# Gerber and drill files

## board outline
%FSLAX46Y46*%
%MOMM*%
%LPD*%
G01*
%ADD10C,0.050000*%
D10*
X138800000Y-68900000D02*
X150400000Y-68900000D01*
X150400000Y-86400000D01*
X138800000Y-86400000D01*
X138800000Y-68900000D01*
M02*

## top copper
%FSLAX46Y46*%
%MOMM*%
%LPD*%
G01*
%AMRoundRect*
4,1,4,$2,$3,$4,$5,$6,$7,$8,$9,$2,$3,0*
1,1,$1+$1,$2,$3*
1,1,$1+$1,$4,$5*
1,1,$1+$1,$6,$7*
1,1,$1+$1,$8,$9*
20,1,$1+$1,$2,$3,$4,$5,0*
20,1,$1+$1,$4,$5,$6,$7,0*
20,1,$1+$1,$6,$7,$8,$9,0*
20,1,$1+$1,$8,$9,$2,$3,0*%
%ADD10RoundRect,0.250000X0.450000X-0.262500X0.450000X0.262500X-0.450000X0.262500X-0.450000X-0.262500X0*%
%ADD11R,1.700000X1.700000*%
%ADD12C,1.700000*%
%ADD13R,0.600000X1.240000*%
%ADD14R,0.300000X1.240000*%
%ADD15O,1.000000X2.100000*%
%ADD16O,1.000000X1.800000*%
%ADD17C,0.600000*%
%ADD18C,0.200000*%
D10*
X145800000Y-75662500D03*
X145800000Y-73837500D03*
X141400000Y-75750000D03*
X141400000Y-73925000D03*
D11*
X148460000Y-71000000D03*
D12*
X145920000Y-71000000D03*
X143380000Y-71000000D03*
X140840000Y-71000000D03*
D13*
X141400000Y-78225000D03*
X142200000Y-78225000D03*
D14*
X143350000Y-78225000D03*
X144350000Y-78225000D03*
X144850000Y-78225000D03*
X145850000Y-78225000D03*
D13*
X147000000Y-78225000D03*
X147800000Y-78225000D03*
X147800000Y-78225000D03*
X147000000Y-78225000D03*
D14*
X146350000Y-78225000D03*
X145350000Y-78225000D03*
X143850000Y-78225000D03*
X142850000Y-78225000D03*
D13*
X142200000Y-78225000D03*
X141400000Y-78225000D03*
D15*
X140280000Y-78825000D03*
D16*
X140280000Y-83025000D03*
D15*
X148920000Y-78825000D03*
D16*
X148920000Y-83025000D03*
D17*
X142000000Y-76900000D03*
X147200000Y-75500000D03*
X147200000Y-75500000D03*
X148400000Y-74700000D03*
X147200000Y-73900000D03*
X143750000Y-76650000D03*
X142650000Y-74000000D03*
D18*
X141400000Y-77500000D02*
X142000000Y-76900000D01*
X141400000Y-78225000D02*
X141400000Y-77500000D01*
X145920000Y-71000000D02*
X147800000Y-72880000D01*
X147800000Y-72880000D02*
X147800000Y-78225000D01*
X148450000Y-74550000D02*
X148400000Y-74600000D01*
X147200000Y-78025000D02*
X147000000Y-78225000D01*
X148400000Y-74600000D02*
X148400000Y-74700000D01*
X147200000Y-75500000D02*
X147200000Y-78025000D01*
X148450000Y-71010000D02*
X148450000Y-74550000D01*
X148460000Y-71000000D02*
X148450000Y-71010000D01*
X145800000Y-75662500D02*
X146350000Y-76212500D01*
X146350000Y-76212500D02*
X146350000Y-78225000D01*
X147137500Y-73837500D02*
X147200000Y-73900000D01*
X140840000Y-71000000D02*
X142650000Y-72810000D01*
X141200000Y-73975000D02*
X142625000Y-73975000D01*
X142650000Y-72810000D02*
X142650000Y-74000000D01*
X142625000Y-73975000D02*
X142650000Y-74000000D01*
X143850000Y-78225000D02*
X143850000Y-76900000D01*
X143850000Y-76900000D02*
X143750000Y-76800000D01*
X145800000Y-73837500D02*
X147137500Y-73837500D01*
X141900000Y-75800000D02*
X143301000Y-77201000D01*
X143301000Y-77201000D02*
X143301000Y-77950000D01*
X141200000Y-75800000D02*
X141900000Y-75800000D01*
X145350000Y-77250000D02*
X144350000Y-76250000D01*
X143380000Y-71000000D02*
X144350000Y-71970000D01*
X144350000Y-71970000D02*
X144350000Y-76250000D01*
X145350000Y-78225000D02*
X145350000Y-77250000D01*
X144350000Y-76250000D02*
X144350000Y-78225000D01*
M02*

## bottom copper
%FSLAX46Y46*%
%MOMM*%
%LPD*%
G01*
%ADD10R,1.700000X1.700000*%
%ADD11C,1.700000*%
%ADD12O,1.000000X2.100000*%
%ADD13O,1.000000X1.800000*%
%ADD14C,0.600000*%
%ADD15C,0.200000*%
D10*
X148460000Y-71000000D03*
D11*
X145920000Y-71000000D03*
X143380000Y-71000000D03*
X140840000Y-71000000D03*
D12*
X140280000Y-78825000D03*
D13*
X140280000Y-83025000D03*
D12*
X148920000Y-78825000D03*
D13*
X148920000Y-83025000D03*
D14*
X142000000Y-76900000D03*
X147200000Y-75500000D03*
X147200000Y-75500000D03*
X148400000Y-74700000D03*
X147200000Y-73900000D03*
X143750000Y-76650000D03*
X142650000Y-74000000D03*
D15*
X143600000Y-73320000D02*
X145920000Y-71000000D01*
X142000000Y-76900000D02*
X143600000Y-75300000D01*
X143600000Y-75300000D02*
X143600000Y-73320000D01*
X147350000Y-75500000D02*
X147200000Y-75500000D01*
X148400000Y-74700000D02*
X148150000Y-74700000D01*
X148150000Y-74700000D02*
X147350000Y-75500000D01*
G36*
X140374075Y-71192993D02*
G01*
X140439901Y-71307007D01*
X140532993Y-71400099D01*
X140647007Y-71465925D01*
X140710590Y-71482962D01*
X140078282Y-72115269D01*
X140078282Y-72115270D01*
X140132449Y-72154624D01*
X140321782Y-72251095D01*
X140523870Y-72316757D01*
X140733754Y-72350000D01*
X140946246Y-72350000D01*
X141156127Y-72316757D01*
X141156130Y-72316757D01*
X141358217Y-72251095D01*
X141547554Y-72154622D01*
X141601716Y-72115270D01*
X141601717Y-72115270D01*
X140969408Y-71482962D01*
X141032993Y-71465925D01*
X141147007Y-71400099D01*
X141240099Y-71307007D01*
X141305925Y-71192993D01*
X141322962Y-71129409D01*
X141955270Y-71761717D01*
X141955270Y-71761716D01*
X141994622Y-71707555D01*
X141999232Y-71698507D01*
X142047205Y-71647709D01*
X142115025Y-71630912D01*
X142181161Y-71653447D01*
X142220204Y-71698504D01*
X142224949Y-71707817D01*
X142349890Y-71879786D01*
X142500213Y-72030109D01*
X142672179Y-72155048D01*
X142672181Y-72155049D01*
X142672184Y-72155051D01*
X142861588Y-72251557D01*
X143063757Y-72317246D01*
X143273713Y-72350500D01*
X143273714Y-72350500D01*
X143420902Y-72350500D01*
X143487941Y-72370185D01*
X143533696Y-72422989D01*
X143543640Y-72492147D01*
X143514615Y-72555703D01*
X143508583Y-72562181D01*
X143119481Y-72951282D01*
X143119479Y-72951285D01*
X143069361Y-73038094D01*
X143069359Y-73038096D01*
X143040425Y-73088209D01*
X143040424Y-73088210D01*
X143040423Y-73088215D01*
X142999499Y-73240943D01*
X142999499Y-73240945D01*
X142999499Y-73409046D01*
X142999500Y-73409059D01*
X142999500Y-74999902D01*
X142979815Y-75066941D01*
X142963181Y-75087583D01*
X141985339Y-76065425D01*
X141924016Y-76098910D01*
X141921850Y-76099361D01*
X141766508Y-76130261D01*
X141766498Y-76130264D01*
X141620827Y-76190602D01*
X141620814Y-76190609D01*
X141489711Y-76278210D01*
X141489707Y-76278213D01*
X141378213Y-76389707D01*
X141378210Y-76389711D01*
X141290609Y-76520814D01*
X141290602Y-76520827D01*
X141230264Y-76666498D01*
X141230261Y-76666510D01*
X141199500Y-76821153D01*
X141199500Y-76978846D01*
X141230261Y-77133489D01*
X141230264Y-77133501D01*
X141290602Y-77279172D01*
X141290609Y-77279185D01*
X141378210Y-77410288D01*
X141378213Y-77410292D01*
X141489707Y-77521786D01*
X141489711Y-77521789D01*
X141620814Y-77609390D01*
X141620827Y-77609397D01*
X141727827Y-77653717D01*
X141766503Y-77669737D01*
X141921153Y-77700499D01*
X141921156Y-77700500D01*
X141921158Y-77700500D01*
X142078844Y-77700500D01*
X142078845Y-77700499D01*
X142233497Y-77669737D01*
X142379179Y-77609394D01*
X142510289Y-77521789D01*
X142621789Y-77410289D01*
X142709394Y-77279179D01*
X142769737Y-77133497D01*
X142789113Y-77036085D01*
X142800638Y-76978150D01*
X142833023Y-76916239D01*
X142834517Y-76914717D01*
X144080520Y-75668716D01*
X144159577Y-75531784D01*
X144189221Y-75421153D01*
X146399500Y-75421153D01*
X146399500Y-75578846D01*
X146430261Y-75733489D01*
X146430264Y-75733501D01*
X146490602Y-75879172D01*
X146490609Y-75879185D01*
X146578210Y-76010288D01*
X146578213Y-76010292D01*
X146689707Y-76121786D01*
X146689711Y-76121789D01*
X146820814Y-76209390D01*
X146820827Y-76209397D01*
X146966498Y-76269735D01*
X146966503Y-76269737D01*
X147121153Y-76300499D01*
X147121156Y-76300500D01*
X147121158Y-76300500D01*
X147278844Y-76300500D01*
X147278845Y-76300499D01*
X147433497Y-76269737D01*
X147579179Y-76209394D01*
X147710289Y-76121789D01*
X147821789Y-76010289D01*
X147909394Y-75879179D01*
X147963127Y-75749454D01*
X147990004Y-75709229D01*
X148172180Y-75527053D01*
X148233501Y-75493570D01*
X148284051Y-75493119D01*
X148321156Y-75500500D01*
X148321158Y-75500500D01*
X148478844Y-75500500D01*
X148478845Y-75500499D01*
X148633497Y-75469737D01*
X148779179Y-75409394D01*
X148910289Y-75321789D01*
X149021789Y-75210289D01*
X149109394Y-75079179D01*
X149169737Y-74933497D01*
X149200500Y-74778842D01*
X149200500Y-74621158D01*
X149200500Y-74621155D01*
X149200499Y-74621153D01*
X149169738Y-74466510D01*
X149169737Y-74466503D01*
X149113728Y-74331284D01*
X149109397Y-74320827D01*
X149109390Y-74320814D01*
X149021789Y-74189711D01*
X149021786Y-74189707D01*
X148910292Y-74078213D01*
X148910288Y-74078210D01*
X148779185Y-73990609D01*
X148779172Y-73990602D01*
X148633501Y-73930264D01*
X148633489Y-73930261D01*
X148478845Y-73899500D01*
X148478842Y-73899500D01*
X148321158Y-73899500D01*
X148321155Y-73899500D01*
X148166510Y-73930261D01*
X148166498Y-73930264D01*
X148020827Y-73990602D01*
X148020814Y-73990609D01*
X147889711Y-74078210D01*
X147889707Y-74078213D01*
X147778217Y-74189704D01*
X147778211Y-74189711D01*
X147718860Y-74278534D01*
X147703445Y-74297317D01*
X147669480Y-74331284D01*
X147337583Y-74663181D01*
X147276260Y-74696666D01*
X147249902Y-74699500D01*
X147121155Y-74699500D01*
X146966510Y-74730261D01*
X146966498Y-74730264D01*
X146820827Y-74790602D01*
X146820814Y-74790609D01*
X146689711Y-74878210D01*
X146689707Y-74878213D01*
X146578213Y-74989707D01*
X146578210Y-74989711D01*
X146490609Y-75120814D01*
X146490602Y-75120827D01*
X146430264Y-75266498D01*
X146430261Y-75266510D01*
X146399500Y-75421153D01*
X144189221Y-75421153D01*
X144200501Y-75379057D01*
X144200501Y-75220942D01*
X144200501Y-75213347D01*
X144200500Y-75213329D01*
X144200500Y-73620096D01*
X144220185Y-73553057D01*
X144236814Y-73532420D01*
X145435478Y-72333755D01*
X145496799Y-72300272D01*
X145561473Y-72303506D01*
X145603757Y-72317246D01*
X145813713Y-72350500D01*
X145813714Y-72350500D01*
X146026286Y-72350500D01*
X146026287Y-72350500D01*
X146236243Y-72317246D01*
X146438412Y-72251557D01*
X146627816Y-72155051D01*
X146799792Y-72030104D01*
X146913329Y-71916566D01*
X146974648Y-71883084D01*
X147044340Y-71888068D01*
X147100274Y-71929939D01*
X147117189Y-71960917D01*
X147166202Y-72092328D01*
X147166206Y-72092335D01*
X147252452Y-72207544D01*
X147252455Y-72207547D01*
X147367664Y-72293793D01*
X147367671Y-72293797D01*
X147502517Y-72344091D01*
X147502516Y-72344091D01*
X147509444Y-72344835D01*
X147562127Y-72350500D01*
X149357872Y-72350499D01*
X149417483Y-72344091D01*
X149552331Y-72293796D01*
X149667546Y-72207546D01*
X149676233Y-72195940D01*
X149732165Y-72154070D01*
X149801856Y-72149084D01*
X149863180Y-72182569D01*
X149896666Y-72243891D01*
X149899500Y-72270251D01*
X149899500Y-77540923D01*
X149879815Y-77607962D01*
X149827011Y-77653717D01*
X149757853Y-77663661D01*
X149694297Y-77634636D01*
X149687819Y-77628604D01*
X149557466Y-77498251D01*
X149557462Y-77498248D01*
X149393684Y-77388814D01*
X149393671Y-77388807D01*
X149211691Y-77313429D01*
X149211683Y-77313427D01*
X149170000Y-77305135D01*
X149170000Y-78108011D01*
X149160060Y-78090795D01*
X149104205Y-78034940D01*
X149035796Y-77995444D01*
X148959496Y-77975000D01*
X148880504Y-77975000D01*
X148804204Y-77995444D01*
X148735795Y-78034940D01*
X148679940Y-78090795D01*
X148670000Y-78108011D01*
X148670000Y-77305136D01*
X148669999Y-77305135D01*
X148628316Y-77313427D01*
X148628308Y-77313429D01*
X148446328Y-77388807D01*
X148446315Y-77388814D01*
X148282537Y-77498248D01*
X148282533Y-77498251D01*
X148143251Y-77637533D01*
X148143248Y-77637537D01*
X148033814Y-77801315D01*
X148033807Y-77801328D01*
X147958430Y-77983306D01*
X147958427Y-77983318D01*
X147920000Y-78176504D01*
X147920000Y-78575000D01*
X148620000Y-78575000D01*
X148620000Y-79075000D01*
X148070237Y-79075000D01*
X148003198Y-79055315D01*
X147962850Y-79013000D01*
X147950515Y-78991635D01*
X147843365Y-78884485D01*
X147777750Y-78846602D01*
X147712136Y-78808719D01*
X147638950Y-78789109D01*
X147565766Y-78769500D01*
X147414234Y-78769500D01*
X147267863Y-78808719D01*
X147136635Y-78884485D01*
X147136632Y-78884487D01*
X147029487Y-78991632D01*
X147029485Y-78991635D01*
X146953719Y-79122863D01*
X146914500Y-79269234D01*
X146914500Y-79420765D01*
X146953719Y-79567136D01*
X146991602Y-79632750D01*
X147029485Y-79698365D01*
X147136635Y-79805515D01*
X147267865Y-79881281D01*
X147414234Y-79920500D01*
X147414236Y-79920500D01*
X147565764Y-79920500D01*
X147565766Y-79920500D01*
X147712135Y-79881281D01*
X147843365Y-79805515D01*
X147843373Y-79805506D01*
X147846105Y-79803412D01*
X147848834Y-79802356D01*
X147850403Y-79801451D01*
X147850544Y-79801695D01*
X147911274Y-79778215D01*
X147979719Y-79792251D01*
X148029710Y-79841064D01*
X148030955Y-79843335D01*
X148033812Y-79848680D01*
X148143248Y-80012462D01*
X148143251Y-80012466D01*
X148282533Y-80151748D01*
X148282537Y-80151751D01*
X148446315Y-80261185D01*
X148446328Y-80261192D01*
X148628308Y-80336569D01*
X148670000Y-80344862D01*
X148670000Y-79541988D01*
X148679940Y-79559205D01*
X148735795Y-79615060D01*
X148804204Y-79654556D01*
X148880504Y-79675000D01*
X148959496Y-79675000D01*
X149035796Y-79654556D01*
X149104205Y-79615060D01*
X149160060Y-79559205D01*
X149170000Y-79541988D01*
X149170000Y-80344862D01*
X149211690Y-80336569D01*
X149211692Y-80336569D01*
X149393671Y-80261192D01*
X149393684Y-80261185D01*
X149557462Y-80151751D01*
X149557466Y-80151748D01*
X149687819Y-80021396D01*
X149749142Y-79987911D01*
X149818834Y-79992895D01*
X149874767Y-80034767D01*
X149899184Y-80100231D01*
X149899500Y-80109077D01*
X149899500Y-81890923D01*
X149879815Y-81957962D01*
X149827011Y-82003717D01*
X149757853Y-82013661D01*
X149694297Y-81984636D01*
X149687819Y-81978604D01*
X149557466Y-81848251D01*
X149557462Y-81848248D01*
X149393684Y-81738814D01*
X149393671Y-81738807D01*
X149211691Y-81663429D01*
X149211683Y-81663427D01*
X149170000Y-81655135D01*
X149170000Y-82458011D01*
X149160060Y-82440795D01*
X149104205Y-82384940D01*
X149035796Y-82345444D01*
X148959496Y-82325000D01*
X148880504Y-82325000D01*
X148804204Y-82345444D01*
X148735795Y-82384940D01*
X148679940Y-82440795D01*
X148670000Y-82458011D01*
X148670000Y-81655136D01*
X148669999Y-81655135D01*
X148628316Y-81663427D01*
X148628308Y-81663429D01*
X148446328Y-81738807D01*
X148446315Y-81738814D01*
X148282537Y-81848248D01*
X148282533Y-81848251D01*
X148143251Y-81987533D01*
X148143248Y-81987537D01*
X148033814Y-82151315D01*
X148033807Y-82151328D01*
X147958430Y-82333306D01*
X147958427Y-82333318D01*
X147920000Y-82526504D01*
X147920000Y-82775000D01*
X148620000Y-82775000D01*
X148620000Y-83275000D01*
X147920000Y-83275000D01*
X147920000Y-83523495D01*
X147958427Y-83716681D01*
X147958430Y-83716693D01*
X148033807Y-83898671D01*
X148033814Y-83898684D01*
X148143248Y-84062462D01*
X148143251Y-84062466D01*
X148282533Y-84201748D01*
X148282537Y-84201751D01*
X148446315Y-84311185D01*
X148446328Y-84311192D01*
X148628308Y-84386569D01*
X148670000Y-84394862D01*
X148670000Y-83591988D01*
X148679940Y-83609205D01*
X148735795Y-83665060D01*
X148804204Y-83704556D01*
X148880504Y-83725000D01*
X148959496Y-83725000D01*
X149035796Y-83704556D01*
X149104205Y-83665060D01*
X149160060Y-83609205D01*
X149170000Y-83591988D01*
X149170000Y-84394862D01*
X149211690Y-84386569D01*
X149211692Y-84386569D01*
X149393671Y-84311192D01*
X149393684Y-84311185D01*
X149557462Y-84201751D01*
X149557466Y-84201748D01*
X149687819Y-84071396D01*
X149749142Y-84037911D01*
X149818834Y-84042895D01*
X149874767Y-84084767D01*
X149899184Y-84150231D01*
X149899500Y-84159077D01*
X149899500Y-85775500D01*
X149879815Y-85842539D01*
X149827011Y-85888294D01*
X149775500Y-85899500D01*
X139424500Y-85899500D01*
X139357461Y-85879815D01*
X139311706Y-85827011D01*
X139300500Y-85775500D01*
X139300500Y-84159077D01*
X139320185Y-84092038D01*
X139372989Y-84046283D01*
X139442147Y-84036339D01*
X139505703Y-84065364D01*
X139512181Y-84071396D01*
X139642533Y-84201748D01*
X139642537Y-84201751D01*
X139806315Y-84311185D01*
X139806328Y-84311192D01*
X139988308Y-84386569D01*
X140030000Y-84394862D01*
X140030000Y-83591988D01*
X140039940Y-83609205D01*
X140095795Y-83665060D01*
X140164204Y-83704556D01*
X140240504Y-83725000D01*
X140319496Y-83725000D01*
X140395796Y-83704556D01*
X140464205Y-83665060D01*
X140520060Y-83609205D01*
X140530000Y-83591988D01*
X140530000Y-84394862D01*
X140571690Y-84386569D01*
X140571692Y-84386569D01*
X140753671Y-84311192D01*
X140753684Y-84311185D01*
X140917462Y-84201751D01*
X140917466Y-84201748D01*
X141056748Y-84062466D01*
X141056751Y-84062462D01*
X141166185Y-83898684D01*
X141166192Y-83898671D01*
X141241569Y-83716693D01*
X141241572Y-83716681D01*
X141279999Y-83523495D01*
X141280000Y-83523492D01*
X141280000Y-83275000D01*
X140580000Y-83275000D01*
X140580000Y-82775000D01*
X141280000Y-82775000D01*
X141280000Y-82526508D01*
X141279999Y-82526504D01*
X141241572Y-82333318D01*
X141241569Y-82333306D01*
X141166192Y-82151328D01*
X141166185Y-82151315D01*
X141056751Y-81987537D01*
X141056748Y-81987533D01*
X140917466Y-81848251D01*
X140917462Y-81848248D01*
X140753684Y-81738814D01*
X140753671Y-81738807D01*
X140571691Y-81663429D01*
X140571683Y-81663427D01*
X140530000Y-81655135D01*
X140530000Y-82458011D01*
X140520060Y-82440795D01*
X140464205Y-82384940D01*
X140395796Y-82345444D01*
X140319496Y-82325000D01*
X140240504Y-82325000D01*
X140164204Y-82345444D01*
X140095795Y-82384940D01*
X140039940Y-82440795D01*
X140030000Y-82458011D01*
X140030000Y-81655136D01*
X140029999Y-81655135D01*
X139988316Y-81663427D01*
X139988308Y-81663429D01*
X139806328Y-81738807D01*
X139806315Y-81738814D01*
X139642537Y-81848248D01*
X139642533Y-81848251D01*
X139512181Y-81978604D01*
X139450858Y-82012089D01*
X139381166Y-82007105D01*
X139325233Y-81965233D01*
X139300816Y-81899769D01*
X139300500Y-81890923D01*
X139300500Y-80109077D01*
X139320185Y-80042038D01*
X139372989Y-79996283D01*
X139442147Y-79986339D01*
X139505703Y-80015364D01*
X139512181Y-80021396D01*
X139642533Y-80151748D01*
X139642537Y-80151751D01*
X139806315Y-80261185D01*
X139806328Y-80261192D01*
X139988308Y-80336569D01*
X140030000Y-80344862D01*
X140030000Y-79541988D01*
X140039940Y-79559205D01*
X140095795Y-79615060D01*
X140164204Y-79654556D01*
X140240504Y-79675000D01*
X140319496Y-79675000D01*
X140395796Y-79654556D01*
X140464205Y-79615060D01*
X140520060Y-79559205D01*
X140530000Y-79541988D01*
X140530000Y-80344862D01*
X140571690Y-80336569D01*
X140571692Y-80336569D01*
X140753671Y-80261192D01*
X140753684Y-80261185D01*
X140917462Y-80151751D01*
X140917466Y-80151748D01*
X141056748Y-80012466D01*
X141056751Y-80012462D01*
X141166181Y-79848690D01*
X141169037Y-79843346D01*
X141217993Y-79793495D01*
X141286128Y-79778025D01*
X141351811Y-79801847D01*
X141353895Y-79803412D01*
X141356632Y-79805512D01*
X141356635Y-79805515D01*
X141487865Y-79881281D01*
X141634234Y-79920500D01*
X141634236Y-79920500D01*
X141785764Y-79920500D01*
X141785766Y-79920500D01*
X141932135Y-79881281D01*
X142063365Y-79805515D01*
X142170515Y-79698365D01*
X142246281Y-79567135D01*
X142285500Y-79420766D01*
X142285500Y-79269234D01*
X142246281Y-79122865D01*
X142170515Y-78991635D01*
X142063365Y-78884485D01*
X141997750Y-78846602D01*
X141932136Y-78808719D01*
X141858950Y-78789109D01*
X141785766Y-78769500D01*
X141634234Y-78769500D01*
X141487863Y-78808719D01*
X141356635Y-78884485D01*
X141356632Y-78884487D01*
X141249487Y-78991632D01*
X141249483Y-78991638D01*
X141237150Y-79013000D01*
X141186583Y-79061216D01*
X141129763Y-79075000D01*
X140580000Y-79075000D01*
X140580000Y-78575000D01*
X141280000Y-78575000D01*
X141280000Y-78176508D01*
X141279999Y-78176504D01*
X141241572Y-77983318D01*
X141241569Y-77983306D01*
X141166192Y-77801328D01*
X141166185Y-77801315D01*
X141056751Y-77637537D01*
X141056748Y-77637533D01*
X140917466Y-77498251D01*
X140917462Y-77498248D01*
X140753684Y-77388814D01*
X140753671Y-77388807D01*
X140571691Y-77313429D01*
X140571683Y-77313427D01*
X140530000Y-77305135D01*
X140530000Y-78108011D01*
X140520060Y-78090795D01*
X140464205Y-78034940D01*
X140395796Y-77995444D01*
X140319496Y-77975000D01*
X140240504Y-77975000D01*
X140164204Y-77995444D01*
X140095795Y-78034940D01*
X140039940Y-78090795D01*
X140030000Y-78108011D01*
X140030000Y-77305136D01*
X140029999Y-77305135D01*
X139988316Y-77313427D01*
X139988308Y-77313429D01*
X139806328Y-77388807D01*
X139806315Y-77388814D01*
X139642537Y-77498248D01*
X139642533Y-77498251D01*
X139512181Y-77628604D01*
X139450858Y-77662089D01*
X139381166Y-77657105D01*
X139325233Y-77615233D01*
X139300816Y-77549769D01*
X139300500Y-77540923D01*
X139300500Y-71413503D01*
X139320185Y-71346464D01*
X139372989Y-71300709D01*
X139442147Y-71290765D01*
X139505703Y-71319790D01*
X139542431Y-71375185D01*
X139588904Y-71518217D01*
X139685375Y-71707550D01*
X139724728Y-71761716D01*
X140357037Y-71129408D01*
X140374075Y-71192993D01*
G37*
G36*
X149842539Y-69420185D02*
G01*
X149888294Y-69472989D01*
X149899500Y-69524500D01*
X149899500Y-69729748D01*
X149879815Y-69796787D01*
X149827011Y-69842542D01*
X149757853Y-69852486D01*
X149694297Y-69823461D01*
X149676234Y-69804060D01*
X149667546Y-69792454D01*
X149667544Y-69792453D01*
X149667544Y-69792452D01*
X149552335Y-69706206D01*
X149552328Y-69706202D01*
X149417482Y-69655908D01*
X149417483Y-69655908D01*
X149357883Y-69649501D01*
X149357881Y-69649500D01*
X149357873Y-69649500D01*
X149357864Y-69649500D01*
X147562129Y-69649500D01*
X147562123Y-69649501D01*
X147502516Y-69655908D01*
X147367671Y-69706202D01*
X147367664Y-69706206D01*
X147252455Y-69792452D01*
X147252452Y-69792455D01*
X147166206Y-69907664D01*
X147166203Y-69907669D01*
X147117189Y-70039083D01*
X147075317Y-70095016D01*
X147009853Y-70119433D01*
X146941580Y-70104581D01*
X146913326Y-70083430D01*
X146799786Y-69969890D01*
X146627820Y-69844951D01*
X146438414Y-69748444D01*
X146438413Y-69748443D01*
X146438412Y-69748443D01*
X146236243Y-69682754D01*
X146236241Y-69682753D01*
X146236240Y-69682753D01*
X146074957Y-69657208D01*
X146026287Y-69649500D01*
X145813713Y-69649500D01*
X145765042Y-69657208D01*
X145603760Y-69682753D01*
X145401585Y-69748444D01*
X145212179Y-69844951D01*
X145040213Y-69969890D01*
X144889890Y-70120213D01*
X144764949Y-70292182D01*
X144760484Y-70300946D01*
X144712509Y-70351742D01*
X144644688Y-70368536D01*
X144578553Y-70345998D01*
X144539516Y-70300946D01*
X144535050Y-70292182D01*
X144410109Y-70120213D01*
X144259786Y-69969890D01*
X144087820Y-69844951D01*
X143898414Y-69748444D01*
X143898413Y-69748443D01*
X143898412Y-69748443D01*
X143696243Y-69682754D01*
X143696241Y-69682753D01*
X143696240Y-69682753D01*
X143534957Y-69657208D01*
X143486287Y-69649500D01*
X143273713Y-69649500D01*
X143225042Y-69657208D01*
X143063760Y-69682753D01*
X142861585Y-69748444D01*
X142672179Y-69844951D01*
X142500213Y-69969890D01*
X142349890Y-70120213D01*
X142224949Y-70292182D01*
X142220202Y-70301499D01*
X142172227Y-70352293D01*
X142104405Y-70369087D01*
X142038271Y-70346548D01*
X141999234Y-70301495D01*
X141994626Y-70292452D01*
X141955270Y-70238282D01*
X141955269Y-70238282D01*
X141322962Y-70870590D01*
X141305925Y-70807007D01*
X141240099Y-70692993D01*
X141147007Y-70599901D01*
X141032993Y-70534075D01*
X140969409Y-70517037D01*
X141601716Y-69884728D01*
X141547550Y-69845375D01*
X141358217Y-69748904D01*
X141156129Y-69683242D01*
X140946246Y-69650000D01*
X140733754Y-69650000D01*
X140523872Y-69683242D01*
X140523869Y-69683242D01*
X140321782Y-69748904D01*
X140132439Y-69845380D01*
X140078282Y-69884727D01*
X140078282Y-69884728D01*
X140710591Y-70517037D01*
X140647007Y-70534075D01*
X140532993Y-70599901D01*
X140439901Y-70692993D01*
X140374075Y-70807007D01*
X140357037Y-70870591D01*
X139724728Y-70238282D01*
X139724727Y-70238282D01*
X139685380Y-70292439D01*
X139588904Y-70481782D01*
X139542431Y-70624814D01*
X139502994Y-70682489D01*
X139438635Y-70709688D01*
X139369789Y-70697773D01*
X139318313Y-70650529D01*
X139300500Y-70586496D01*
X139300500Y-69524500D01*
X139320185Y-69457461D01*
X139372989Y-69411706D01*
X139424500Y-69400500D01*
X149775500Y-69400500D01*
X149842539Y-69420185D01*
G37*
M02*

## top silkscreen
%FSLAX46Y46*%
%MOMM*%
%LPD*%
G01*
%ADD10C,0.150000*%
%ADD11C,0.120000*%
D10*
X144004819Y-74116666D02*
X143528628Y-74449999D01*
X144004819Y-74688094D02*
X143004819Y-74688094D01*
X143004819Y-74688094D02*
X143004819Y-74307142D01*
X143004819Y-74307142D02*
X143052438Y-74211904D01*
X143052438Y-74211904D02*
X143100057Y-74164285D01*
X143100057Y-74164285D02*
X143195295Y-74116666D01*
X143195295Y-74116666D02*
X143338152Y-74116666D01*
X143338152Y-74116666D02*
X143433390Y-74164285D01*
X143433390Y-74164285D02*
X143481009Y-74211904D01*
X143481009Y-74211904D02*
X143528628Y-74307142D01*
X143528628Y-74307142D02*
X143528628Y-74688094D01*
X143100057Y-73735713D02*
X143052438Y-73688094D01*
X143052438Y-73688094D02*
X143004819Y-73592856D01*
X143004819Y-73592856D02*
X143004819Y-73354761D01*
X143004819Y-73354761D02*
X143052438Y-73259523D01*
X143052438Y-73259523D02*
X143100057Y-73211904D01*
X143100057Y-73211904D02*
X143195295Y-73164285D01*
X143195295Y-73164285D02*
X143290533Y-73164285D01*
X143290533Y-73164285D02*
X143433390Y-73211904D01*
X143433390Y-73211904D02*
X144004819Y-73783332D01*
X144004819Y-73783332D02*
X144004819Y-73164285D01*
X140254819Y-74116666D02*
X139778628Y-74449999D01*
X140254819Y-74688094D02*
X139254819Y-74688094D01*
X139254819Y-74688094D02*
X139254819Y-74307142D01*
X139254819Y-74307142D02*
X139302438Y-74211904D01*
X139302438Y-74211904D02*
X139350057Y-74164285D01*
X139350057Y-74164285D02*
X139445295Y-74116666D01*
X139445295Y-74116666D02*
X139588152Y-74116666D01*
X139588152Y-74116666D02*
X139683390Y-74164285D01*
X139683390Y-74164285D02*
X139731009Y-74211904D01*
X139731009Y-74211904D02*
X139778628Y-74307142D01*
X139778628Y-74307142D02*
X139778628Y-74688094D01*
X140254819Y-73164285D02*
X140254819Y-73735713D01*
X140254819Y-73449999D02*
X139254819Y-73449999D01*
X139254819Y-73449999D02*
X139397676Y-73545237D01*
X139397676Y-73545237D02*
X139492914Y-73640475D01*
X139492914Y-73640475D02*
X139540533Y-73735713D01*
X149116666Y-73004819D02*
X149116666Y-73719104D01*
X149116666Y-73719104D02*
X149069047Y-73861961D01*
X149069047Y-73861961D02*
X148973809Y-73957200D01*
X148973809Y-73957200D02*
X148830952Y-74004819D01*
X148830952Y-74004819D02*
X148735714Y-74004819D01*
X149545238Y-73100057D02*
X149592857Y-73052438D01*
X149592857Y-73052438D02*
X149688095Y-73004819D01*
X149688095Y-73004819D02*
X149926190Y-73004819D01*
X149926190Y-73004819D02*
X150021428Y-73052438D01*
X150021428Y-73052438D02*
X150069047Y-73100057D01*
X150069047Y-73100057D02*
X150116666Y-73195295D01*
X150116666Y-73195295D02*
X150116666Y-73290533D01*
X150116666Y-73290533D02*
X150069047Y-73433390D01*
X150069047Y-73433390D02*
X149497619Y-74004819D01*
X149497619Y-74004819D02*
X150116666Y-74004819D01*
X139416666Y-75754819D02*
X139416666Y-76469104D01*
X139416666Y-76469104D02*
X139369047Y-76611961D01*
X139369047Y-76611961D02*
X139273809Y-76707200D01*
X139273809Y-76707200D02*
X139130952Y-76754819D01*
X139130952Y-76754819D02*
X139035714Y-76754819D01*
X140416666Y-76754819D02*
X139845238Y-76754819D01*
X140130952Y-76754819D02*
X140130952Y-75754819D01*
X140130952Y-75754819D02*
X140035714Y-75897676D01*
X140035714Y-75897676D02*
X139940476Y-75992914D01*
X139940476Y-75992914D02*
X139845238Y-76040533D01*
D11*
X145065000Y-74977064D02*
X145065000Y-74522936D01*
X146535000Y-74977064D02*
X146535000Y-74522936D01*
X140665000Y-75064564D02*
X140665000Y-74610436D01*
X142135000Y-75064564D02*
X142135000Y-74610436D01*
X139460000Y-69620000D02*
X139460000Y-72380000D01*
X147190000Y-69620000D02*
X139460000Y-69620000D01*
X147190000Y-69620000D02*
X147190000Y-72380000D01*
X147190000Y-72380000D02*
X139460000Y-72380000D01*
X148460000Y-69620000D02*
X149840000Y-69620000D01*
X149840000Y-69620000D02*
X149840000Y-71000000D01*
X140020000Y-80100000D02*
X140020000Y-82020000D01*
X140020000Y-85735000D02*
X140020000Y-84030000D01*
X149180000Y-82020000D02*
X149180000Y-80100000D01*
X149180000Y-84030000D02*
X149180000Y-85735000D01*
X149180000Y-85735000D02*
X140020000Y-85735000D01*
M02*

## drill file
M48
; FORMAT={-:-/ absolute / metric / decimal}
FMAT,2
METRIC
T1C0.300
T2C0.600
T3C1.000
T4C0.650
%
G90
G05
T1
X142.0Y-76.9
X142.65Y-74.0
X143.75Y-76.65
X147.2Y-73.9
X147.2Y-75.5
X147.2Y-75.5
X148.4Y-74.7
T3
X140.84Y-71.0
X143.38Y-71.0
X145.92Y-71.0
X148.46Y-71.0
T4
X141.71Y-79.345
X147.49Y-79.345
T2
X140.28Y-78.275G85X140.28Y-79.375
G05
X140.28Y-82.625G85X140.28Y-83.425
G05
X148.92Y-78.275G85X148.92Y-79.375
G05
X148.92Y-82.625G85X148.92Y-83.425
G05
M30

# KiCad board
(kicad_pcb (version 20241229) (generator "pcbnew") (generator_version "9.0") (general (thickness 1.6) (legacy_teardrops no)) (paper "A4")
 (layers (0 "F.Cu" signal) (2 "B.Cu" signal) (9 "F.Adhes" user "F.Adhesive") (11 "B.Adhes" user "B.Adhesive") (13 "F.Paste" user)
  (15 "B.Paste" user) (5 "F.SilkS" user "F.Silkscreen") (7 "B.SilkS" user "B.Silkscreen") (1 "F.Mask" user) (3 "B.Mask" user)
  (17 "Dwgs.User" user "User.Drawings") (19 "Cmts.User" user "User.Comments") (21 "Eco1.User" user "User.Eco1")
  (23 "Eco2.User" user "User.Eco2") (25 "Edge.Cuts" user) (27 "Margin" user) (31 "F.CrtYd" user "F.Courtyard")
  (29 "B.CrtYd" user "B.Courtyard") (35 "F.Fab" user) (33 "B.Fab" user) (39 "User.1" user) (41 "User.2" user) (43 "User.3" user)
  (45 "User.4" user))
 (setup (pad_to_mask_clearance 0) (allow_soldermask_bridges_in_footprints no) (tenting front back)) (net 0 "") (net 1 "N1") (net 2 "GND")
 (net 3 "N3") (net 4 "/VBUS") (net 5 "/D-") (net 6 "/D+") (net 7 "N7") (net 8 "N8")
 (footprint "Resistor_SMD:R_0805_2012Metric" (layer "F.Cu") (at 145.8 74.75 90)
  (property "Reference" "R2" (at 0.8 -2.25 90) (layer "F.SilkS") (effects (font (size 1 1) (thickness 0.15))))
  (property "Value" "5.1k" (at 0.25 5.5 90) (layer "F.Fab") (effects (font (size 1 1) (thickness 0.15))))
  (fp_line (start -0.227064 -0.735) (end 0.227064 -0.735) (stroke (width 0.12) (type solid)) (layer "F.SilkS"))
  (fp_line (start -0.227064 0.735) (end 0.227064 0.735) (stroke (width 0.12) (type solid)) (layer "F.SilkS"))
  (pad "1" smd roundrect (at -0.9125 0 90) (size 1.025 1.4) (layers "F.Cu" "F.Mask" "F.Paste") (roundrect_rratio 0.243902) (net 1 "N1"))
  (pad "2" smd roundrect (at 0.9125 0 90) (size 1.025 1.4) (layers "F.Cu" "F.Mask" "F.Paste") (roundrect_rratio 0.243902) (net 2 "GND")))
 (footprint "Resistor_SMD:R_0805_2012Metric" (layer "F.Cu") (at 141.4 74.8375 90)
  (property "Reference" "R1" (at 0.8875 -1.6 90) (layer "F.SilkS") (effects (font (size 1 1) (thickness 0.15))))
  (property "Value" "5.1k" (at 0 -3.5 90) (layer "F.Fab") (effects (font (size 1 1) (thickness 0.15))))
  (fp_line (start -0.227064 -0.735) (end 0.227064 -0.735) (stroke (width 0.12) (type solid)) (layer "F.SilkS"))
  (fp_line (start -0.227064 0.735) (end 0.227064 0.735) (stroke (width 0.12) (type solid)) (layer "F.SilkS"))
  (pad "1" smd roundrect (at -0.9125 0 90) (size 1.025 1.4) (layers "F.Cu" "F.Mask" "F.Paste") (roundrect_rratio 0.243902) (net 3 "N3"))
  (pad "2" smd roundrect (at 0.9125 0 90) (size 1.025 1.4) (layers "F.Cu" "F.Mask" "F.Paste") (roundrect_rratio 0.243902) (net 2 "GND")))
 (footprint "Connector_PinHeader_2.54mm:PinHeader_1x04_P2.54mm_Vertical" (layer "F.Cu") (at 148.46 71 -90)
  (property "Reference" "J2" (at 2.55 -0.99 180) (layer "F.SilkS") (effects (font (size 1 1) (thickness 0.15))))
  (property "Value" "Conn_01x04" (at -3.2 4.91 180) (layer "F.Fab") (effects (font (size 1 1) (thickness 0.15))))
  (fp_line (start -1.38 9) (end 1.38 9) (stroke (width 0.12) (type solid)) (layer "F.SilkS"))
  (fp_line (start -1.38 1.27) (end -1.38 9) (stroke (width 0.12) (type solid)) (layer "F.SilkS"))
  (fp_line (start -1.38 1.27) (end 1.38 1.27) (stroke (width 0.12) (type solid)) (layer "F.SilkS"))
  (fp_line (start 1.38 1.27) (end 1.38 9) (stroke (width 0.12) (type solid)) (layer "F.SilkS"))
  (fp_line (start -1.38 0) (end -1.38 -1.38) (stroke (width 0.12) (type solid)) (layer "F.SilkS"))
  (fp_line (start -1.38 -1.38) (end 0 -1.38) (stroke (width 0.12) (type solid)) (layer "F.SilkS"))
  (pad "1" thru_hole rect (at 0 0 270) (size 1.7 1.7) (drill 1) (layers "*.Cu" "*.Mask") (remove_unused_layers no) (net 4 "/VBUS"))
  (pad "2" thru_hole circle (at 0 2.54 270) (size 1.7 1.7) (drill 1) (layers "*.Cu" "*.Mask") (remove_unused_layers no) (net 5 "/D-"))
  (pad "3" thru_hole circle (at 0 5.08 270) (size 1.7 1.7) (drill 1) (layers "*.Cu" "*.Mask") (remove_unused_layers no) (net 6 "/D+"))
  (pad "4" thru_hole circle (at 0 7.62 270) (size 1.7 1.7) (drill 1) (layers "*.Cu" "*.Mask") (remove_unused_layers no) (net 2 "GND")))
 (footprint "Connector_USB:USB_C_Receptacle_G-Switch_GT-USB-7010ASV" (layer "F.Cu") (at 144.6 81.95)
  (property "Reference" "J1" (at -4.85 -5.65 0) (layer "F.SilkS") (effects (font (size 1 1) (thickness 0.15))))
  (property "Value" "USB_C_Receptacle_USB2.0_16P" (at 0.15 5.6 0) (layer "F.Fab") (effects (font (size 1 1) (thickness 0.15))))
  (fp_line (start -4.58 -1.85) (end -4.58 0.07) (stroke (width 0.12) (type solid)) (layer "F.SilkS"))
  (fp_line (start -4.58 3.785) (end -4.58 2.08) (stroke (width 0.12) (type solid)) (layer "F.SilkS"))
  (fp_line (start 4.58 0.07) (end 4.58 -1.85) (stroke (width 0.12) (type solid)) (layer "F.SilkS"))
  (fp_line (start 4.58 2.08) (end 4.58 3.785) (stroke (width 0.12) (type solid)) (layer "F.SilkS"))
  (fp_line (start 4.58 3.785) (end -4.58 3.785) (stroke (width 0.12) (type solid)) (layer "F.SilkS"))
  (pad "" np_thru_hole circle (at -2.89 -2.605) (size 0.65 0.65) (drill 0.65) (layers "*.Cu" "*.Mask"))
  (pad "" np_thru_hole circle (at 2.89 -2.605) (size 0.65 0.65) (drill 0.65) (layers "*.Cu" "*.Mask"))
  (pad "A1" smd rect (at -3.2 -3.725) (size 0.6 1.24) (layers "F.Cu" "F.Mask" "F.Paste") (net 5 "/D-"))
  (pad "A4" smd rect (at -2.4 -3.725) (size 0.6 1.24) (layers "F.Cu" "F.Mask" "F.Paste") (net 4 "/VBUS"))
  (pad "A5" smd rect (at -1.25 -3.725) (size 0.3 1.24) (layers "F.Cu" "F.Mask" "F.Paste") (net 3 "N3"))
  (pad "A6" smd rect (at -0.25 -3.725) (size 0.3 1.24) (layers "F.Cu" "F.Mask" "F.Paste") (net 6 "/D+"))
  (pad "A7" smd rect (at 0.25 -3.725) (size 0.3 1.24) (layers "F.Cu" "F.Mask" "F.Paste") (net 2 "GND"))
  (pad "A8" smd rect (at 1.25 -3.725) (size 0.3 1.24) (layers "F.Cu" "F.Mask" "F.Paste") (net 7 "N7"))
  (pad "A9" smd rect (at 2.4 -3.725) (size 0.6 1.24) (layers "F.Cu" "F.Mask" "F.Paste") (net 4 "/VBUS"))
  (pad "A12" smd rect (at 3.2 -3.725) (size 0.6 1.24) (layers "F.Cu" "F.Mask" "F.Paste") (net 5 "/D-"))
  (pad "B1" smd rect (at 3.2 -3.725) (size 0.6 1.24) (layers "F.Cu" "F.Mask" "F.Paste") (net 5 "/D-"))
  (pad "B4" smd rect (at 2.4 -3.725) (size 0.6 1.24) (layers "F.Cu" "F.Mask" "F.Paste") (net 4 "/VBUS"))
  (pad "B5" smd rect (at 1.75 -3.725) (size 0.3 1.24) (layers "F.Cu" "F.Mask" "F.Paste") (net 1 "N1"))
  (pad "B6" smd rect (at 0.75 -3.725) (size 0.3 1.24) (layers "F.Cu" "F.Mask" "F.Paste") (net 6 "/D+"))
  (pad "B7" smd rect (at -0.75 -3.725) (size 0.3 1.24) (layers "F.Cu" "F.Mask" "F.Paste") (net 2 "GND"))
  (pad "B8" smd rect (at -1.75 -3.725) (size 0.3 1.24) (layers "F.Cu" "F.Mask" "F.Paste") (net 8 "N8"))
  (pad "B9" smd rect (at -2.4 -3.725) (size 0.6 1.24) (layers "F.Cu" "F.Mask" "F.Paste") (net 4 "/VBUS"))
  (pad "B12" smd rect (at -3.2 -3.725) (size 0.6 1.24) (layers "F.Cu" "F.Mask" "F.Paste") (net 5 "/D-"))
  (pad "S1" thru_hole oval (at -4.32 -3.125) (size 1 2.1) (drill oval 0.6 1.7) (layers "*.Cu" "*.Mask") (remove_unused_layers no)
   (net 2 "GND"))
  (pad "S1" thru_hole oval (at -4.32 1.075) (size 1 1.8) (drill oval 0.6 1.4) (layers "*.Cu" "*.Mask") (remove_unused_layers no)
   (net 2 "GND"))
  (pad "S1" thru_hole oval (at 4.32 -3.125) (size 1 2.1) (drill oval 0.6 1.7) (layers "*.Cu" "*.Mask") (remove_unused_layers no)
   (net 2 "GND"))
  (pad "S1" thru_hole oval (at 4.32 1.075) (size 1 1.8) (drill oval 0.6 1.4) (layers "*.Cu" "*.Mask") (remove_unused_layers no)
   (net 2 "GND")))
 (gr_rect (start 138.8 68.9) (end 150.4 86.4) (stroke (width 0.05) (type default)) (fill no) (layer "Edge.Cuts"))
 (segment (start 141.4 77.5) (end 142 76.9) (width 0.2) (layer "F.Cu") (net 5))
 (segment (start 141.4 78.225) (end 141.4 77.5) (width 0.2) (layer "F.Cu") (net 5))
 (segment (start 145.92 71) (end 147.8 72.88) (width 0.2) (layer "F.Cu") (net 5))
 (segment (start 147.8 72.88) (end 147.8 78.225) (width 0.2) (layer "F.Cu") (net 5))
 (via (at 142 76.9) (size 0.6) (drill 0.3) (layers "F.Cu" "B.Cu") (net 5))
 (segment (start 143.6 73.32) (end 145.92 71) (width 0.2) (layer "B.Cu") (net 5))
 (segment (start 142 76.9) (end 143.6 75.3) (width 0.2) (layer "B.Cu") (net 5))
 (segment (start 143.6 75.3) (end 143.6 73.32) (width 0.2) (layer "B.Cu") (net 5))
 (segment (start 148.45 74.55) (end 148.4 74.6) (width 0.2) (layer "F.Cu") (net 4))
 (segment (start 147.2 78.025) (end 147 78.225) (width 0.2) (layer "F.Cu") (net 4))
 (segment (start 148.4 74.6) (end 148.4 74.7) (width 0.2) (layer "F.Cu") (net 4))
 (segment (start 147.2 75.5) (end 147.2 78.025) (width 0.2) (layer "F.Cu") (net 4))
 (segment (start 148.45 71.01) (end 148.45 74.55) (width 0.2) (layer "F.Cu") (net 4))
 (segment (start 148.46 71) (end 148.45 71.01) (width 0.2) (layer "F.Cu") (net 4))
 (via (at 147.2 75.5) (size 0.6) (drill 0.3) (layers "F.Cu" "B.Cu") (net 4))
 (via (at 147.2 75.5) (size 0.6) (drill 0.3) (layers "F.Cu" "B.Cu") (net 4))
 (via (at 148.4 74.7) (size 0.6) (drill 0.3) (layers "F.Cu" "B.Cu") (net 4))
 (segment (start 147.35 75.5) (end 147.2 75.5) (width 0.2) (layer "B.Cu") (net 4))
 (segment (start 148.4 74.7) (end 148.15 74.7) (width 0.2) (layer "B.Cu") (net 4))
 (segment (start 148.15 74.7) (end 147.35 75.5) (width 0.2) (layer "B.Cu") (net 4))
 (segment (start 145.8 75.6625) (end 146.35 76.2125) (width 0.2) (layer "F.Cu") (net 1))
 (segment (start 146.35 76.2125) (end 146.35 78.225) (width 0.2) (layer "F.Cu") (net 1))
 (segment (start 147.1375 73.8375) (end 147.2 73.9) (width 0.2) (layer "F.Cu") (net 2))
 (segment (start 140.84 71) (end 142.65 72.81) (width 0.2) (layer "F.Cu") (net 2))
 (segment (start 141.2 73.975) (end 142.625 73.975) (width 0.2) (layer "F.Cu") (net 2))
 (segment (start 142.65 72.81) (end 142.65 74) (width 0.2) (layer "F.Cu") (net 2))
 (segment (start 142.625 73.975) (end 142.65 74) (width 0.2) (layer "F.Cu") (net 2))
 (segment (start 143.85 78.225) (end 143.85 76.9) (width 0.2) (layer "F.Cu") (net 2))
 (segment (start 143.85 76.9) (end 143.75 76.8) (width 0.2) (layer "F.Cu") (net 2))
 (segment (start 145.8 73.8375) (end 147.1375 73.8375) (width 0.2) (layer "F.Cu") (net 2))
 (via (at 147.2 73.9) (size 0.6) (drill 0.3) (layers "F.Cu" "B.Cu") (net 2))
 (via (at 143.75 76.65) (size 0.6) (drill 0.3) (layers "F.Cu" "B.Cu") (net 2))
 (via (at 142.65 74) (size 0.6) (drill 0.3) (layers "F.Cu" "B.Cu") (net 2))
 (segment (start 141.9 75.8) (end 143.301 77.201) (width 0.2) (layer "F.Cu") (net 3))
 (segment (start 143.301 77.201) (end 143.301 77.95) (width 0.2) (layer "F.Cu") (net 3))
 (segment (start 141.2 75.8) (end 141.9 75.8) (width 0.2) (layer "F.Cu") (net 3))
 (segment (start 145.35 77.25) (end 144.35 76.25) (width 0.2) (layer "F.Cu") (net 6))
 (segment (start 143.38 71) (end 144.35 71.97) (width 0.2) (layer "F.Cu") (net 6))
 (segment (start 144.35 71.97) (end 144.35 76.25) (width 0.2) (layer "F.Cu") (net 6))
 (segment (start 145.35 78.225) (end 145.35 77.25) (width 0.2) (layer "F.Cu") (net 6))
 (segment (start 144.35 76.25) (end 144.35 78.225) (width 0.2) (layer "F.Cu") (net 6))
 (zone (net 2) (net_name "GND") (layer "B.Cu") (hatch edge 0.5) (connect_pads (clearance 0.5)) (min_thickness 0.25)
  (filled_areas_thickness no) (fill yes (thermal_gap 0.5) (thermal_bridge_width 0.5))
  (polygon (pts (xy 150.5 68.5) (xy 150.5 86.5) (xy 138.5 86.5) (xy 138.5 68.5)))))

